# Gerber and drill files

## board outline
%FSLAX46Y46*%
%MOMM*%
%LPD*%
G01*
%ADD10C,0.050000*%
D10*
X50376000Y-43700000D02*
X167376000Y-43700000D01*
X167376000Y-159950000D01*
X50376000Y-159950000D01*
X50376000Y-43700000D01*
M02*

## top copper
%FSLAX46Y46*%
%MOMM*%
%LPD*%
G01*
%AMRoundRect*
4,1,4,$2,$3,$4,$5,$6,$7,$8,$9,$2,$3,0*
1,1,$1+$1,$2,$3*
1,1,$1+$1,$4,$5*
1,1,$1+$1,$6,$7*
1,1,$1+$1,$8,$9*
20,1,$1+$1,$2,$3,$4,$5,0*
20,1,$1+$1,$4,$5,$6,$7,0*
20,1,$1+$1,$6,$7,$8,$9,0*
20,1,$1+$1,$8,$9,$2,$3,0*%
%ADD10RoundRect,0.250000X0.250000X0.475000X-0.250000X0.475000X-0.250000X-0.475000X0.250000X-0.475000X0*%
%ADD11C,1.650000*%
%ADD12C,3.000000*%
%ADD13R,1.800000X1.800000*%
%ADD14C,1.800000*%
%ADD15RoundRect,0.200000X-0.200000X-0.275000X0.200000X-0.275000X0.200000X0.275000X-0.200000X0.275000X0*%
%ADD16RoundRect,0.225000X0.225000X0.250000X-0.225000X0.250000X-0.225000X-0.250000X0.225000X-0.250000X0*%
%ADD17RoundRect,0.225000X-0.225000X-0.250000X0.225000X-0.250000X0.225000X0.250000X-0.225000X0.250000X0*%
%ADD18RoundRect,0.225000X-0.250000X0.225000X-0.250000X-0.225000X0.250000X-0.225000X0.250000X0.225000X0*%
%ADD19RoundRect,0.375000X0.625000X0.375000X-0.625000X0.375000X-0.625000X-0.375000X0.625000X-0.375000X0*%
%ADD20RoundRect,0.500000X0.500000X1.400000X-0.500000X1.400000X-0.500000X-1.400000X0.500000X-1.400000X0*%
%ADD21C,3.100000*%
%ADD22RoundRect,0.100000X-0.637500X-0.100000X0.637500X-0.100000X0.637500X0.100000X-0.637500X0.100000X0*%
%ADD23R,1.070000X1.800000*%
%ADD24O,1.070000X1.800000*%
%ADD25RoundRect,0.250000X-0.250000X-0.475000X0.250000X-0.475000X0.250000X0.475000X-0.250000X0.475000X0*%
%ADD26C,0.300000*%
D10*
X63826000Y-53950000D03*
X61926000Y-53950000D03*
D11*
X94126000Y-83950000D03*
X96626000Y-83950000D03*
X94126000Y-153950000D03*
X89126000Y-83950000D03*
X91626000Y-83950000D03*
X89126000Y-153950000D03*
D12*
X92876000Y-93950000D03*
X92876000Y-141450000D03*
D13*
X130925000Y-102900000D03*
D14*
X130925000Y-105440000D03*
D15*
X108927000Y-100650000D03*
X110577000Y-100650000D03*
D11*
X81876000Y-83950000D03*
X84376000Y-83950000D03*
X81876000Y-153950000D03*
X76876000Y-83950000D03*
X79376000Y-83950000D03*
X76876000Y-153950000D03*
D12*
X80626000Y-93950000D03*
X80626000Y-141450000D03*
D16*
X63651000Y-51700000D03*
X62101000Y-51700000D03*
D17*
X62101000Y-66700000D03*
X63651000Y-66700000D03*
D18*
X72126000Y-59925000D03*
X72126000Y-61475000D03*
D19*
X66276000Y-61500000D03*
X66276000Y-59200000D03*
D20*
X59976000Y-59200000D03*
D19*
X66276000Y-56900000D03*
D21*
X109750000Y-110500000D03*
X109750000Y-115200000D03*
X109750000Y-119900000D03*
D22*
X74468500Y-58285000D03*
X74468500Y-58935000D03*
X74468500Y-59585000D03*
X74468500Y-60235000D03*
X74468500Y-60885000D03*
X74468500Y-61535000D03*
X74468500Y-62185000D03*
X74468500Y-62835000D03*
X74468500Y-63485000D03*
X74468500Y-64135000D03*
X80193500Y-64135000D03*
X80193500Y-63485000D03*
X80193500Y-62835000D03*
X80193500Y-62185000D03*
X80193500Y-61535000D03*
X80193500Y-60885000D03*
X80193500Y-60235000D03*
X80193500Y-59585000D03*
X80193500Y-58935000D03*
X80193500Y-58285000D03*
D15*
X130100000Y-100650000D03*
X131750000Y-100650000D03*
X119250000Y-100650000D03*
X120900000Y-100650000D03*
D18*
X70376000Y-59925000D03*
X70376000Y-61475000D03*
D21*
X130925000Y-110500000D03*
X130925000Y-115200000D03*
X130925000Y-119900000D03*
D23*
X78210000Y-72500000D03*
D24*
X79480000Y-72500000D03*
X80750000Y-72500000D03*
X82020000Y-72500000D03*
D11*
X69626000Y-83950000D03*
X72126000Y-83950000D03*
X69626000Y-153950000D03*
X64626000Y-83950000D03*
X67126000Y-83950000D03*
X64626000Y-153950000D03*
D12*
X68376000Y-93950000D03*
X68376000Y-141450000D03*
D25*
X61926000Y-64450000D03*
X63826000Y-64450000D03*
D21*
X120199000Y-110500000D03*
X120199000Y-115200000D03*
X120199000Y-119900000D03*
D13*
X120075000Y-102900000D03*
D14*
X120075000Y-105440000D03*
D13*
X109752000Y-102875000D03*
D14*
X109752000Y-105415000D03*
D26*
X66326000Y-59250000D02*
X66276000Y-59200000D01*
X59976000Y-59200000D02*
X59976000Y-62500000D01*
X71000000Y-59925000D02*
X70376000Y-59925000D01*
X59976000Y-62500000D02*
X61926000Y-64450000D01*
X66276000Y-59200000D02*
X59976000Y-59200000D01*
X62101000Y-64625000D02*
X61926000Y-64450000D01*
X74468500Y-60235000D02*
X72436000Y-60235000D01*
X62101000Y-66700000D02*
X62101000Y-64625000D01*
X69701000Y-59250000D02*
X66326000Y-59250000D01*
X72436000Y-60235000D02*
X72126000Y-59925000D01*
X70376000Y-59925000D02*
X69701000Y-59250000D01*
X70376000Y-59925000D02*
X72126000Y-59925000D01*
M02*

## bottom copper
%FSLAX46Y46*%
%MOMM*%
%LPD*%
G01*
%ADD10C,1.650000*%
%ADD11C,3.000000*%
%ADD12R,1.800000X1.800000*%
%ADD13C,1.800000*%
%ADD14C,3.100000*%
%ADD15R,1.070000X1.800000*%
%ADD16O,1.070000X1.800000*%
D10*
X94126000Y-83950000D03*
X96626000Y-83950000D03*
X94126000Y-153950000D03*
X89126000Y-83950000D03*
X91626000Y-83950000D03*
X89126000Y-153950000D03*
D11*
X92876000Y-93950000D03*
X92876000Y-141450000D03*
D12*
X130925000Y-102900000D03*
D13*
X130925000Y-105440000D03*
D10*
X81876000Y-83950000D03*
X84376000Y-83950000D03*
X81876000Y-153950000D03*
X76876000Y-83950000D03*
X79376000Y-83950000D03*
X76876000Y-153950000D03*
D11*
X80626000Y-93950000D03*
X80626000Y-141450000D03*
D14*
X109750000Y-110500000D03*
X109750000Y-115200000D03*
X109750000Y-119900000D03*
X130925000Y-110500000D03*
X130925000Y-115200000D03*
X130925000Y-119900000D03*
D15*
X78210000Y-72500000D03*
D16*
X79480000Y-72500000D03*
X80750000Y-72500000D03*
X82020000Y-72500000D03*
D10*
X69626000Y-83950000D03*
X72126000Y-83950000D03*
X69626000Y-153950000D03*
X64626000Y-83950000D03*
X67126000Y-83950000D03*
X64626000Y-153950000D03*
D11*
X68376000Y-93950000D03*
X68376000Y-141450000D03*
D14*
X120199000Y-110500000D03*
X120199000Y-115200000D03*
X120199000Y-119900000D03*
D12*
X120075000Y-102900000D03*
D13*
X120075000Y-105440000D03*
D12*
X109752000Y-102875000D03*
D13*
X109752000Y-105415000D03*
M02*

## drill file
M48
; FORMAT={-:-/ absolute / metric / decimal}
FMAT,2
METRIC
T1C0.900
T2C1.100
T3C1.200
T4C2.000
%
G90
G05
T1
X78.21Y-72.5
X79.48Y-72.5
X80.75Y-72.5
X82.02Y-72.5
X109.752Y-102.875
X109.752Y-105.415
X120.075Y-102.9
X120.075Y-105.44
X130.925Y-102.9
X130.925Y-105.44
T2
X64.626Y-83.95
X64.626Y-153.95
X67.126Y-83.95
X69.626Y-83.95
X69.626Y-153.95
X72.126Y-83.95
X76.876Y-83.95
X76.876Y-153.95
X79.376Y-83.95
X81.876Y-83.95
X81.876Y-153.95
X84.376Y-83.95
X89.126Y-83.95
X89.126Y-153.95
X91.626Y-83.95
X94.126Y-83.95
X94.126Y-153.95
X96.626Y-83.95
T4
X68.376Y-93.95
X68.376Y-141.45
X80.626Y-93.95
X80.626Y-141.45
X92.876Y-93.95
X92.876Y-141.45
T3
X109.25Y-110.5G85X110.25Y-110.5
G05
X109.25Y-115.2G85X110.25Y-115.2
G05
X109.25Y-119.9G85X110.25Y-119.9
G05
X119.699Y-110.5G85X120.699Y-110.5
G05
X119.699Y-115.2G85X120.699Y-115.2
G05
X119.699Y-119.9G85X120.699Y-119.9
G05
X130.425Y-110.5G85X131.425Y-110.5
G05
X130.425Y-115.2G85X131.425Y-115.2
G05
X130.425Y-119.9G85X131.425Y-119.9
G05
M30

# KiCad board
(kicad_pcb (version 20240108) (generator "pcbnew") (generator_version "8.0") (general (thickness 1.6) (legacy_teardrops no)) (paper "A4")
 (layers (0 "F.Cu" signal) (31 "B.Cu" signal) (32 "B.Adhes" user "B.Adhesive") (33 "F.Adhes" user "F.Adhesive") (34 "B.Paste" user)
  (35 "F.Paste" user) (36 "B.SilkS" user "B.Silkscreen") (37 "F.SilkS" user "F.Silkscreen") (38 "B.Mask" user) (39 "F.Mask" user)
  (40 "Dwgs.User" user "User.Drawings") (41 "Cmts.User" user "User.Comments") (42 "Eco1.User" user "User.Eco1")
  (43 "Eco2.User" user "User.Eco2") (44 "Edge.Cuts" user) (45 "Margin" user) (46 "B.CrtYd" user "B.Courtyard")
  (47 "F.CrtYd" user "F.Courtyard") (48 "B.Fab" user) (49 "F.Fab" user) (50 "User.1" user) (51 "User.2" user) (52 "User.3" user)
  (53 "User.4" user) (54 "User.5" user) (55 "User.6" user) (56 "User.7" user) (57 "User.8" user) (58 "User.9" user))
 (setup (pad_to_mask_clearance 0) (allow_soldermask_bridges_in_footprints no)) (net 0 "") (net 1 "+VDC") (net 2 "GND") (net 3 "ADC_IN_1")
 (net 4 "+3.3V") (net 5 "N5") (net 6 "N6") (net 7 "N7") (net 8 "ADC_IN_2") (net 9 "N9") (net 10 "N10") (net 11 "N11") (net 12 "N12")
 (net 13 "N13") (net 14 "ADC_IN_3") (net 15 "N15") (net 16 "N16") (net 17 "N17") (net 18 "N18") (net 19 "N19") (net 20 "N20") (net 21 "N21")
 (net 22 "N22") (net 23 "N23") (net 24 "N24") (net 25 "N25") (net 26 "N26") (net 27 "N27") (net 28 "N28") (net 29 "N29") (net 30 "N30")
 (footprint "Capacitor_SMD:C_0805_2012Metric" (layer "F.Cu") (at 62.876 53.95 180)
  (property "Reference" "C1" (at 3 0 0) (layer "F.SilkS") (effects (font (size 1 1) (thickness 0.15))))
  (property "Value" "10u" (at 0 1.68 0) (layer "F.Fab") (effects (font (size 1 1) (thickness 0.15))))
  (pad "1" smd roundrect (at -0.95 0 180) (size 1 1.45) (layers "F.Cu" "F.Paste" "F.Mask") (roundrect_rratio 0.25) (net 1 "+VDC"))
  (pad "2" smd roundrect (at 0.95 0 180) (size 1 1.45) (layers "F.Cu" "F.Paste" "F.Mask") (roundrect_rratio 0.25) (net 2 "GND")))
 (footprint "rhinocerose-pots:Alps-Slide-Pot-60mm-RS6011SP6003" (layer "F.Cu") (at 94.126 83.95 -90)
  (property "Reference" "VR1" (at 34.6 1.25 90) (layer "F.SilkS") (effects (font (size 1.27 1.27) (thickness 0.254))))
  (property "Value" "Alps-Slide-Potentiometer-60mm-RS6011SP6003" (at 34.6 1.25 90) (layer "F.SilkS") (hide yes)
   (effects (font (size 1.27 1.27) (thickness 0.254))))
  (pad "1" thru_hole circle (at 0 0 270) (size 1.65 1.65) (drill 1.1) (layers "*.Cu" "*.Mask") (remove_unused_layers no) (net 2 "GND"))
  (pad "2" thru_hole circle (at 0 -2.5 270) (size 1.65 1.65) (drill 1.1) (layers "*.Cu" "*.Mask") (remove_unused_layers no)
   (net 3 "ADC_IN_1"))
  (pad "3" thru_hole circle (at 70 0 270) (size 1.65 1.65) (drill 1.1) (layers "*.Cu" "*.Mask") (remove_unused_layers no) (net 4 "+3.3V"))
  (pad "L1" thru_hole circle (at 0 5 270) (size 1.65 1.65) (drill 1.1) (layers "*.Cu" "*.Mask") (remove_unused_layers no) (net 2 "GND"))
  (pad "L2" thru_hole circle (at 0 2.5 270) (size 1.65 1.65) (drill 1.1) (layers "*.Cu" "*.Mask") (remove_unused_layers no) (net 2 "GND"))
  (pad "L3" thru_hole circle (at 70 5 270) (size 1.65 1.65) (drill 1.1) (layers "*.Cu" "*.Mask") (remove_unused_layers no) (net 2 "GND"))
  (pad "MH1" thru_hole circle (at 10 1.25 270) (size 3 3) (drill 2) (layers "*.Cu" "*.Mask") (remove_unused_layers no) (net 2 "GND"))
  (pad "MH2" thru_hole circle (at 57.5 1.25 270) (size 3 3) (drill 2) (layers "*.Cu" "*.Mask") (remove_unused_layers no) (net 2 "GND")))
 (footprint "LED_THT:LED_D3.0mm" (layer "F.Cu") (at 130.925 102.9 -90)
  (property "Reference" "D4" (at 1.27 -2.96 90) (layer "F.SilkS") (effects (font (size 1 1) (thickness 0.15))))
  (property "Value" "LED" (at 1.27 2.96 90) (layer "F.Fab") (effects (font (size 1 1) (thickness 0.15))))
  (pad "1" thru_hole rect (at 0 0 270) (size 1.8 1.8) (drill 0.9) (layers "*.Cu" "*.Mask") (remove_unused_layers no) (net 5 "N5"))
  (pad "2" thru_hole circle (at 2.54 0 270) (size 1.8 1.8) (drill 0.9) (layers "*.Cu" "*.Mask") (remove_unused_layers no) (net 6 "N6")))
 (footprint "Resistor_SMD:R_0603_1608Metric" (layer "F.Cu") (at 109.752 100.65)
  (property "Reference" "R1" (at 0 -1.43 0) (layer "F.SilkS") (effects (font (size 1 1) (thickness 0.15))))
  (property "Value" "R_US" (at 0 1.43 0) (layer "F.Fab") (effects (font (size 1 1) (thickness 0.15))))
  (pad "1" smd roundrect (at -0.825 0) (size 0.8 0.95) (layers "F.Cu" "F.Paste" "F.Mask") (roundrect_rratio 0.25) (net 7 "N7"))
  (pad "2" smd roundrect (at 0.825 0) (size 0.8 0.95) (layers "F.Cu" "F.Paste" "F.Mask") (roundrect_rratio 0.25) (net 2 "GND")))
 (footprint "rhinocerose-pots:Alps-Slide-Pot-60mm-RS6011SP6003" (layer "F.Cu") (at 81.876 83.95 -90)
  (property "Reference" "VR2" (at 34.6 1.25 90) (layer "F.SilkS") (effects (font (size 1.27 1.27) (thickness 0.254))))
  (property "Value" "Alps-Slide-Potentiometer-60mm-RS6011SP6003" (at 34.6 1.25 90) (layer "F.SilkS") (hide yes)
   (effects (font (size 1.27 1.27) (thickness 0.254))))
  (pad "1" thru_hole circle (at 0 0 270) (size 1.65 1.65) (drill 1.1) (layers "*.Cu" "*.Mask") (remove_unused_layers no) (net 2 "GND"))
  (pad "2" thru_hole circle (at 0 -2.5 270) (size 1.65 1.65) (drill 1.1) (layers "*.Cu" "*.Mask") (remove_unused_layers no)
   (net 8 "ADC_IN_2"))
  (pad "3" thru_hole circle (at 70 0 270) (size 1.65 1.65) (drill 1.1) (layers "*.Cu" "*.Mask") (remove_unused_layers no) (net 4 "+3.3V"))
  (pad "L1" thru_hole circle (at 0 5 270) (size 1.65 1.65) (drill 1.1) (layers "*.Cu" "*.Mask") (remove_unused_layers no) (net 2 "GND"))
  (pad "L2" thru_hole circle (at 0 2.5 270) (size 1.65 1.65) (drill 1.1) (layers "*.Cu" "*.Mask") (remove_unused_layers no) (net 2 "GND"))
  (pad "L3" thru_hole circle (at 70 5 270) (size 1.65 1.65) (drill 1.1) (layers "*.Cu" "*.Mask") (remove_unused_layers no) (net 2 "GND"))
  (pad "MH1" thru_hole circle (at 10 1.25 270) (size 3 3) (drill 2) (layers "*.Cu" "*.Mask") (remove_unused_layers no) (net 2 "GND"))
  (pad "MH2" thru_hole circle (at 57.5 1.25 270) (size 3 3) (drill 2) (layers "*.Cu" "*.Mask") (remove_unused_layers no) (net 2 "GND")))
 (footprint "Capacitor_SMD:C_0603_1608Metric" (layer "F.Cu") (at 62.876 51.7 180)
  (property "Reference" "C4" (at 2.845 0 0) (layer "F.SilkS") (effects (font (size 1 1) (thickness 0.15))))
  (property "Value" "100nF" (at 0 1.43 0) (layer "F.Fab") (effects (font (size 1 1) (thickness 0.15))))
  (pad "1" smd roundrect (at -0.775 0 180) (size 0.9 0.95) (layers "F.Cu" "F.Paste" "F.Mask") (roundrect_rratio 0.25) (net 1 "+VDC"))
  (pad "2" smd roundrect (at 0.775 0 180) (size 0.9 0.95) (layers "F.Cu" "F.Paste" "F.Mask") (roundrect_rratio 0.25) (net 2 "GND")))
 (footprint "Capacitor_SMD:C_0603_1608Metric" (layer "F.Cu") (at 62.876 66.7)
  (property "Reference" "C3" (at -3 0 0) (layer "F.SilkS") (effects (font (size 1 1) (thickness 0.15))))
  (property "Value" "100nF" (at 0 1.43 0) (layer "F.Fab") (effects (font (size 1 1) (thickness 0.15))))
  (pad "1" smd roundrect (at -0.775 0) (size 0.9 0.95) (layers "F.Cu" "F.Paste" "F.Mask") (roundrect_rratio 0.25) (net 4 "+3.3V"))
  (pad "2" smd roundrect (at 0.775 0) (size 0.9 0.95) (layers "F.Cu" "F.Paste" "F.Mask") (roundrect_rratio 0.25) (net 2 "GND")))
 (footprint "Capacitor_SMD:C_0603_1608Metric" (layer "F.Cu") (at 72.126 60.7 -90)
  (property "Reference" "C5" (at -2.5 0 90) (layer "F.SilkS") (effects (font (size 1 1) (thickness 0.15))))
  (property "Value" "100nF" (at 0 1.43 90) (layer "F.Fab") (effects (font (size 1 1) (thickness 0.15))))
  (pad "1" smd roundrect (at -0.775 0 270) (size 0.9 0.95) (layers "F.Cu" "F.Paste" "F.Mask") (roundrect_rratio 0.25) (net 4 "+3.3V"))
  (pad "2" smd roundrect (at 0.775 0 270) (size 0.9 0.95) (layers "F.Cu" "F.Paste" "F.Mask") (roundrect_rratio 0.25) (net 2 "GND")))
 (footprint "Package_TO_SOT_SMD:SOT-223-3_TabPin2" (layer "F.Cu") (at 63.126 59.2 180)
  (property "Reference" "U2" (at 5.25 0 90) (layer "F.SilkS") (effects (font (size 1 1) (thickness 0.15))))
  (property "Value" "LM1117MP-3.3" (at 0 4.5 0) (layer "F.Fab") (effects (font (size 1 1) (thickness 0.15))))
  (pad "1" smd roundrect (at -3.15 -2.3 180) (size 2 1.5) (layers "F.Cu" "F.Paste" "F.Mask") (roundrect_rratio 0.25) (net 2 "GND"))
  (pad "2" smd roundrect (at -3.15 0 180) (size 2 1.5) (layers "F.Cu" "F.Paste" "F.Mask") (roundrect_rratio 0.25) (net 4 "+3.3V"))
  (pad "2" smd roundrect (at 3.15 0 180) (size 2 3.8) (layers "F.Cu" "F.Paste" "F.Mask") (roundrect_rratio 0.25) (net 4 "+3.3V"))
  (pad "3" smd roundrect (at -3.15 2.3 180) (size 2 1.5) (layers "F.Cu" "F.Paste" "F.Mask") (roundrect_rratio 0.25) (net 1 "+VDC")))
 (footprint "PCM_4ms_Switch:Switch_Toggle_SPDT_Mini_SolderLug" (layer "F.Cu") (at 109.75 115.2)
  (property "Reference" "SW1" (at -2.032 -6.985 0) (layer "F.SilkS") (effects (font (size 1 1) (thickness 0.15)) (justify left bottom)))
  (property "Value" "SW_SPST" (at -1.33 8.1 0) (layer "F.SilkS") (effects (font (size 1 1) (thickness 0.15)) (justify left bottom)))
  (pad "1" thru_hole circle (at 0 -4.7) (size 3.1 3.1) (drill oval 2.2 1.2) (layers "*.Cu" "*.Mask") (remove_unused_layers no) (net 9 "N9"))
  (pad "2" thru_hole circle (at 0 0) (size 3.1 3.1) (drill oval 2.2 1.2) (layers "*.Cu" "*.Mask") (remove_unused_layers no) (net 4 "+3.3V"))
  (pad "3" thru_hole circle (at 0 4.7) (size 3.1 3.1) (drill oval 2.2 1.2) (layers "*.Cu" "*.Mask") (remove_unused_layers no)))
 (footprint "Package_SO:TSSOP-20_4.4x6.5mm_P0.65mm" (layer "F.Cu") (at 77.331 61.21)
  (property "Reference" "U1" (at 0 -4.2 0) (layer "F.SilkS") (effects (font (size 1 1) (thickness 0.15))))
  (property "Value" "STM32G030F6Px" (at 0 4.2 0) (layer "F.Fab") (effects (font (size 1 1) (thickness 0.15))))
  (pad "1" smd roundrect (at -2.8625 -2.925) (size 1.475 0.4) (layers "F.Cu" "F.Paste" "F.Mask") (roundrect_rratio 0.25) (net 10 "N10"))
  (pad "2" smd roundrect (at -2.8625 -2.275) (size 1.475 0.4) (layers "F.Cu" "F.Paste" "F.Mask") (roundrect_rratio 0.25) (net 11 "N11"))
  (pad "3" smd roundrect (at -2.8625 -1.625) (size 1.475 0.4) (layers "F.Cu" "F.Paste" "F.Mask") (roundrect_rratio 0.25) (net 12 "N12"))
  (pad "4" smd roundrect (at -2.8625 -0.975) (size 1.475 0.4) (layers "F.Cu" "F.Paste" "F.Mask") (roundrect_rratio 0.25) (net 4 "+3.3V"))
  (pad "5" smd roundrect (at -2.8625 -0.325) (size 1.475 0.4) (layers "F.Cu" "F.Paste" "F.Mask") (roundrect_rratio 0.25) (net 2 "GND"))
  (pad "6" smd roundrect (at -2.8625 0.325) (size 1.475 0.4) (layers "F.Cu" "F.Paste" "F.Mask") (roundrect_rratio 0.25) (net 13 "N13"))
  (pad "7" smd roundrect (at -2.8625 0.975) (size 1.475 0.4) (layers "F.Cu" "F.Paste" "F.Mask") (roundrect_rratio 0.25) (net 3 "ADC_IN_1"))
  (pad "8" smd roundrect (at -2.8625 1.625) (size 1.475 0.4) (layers "F.Cu" "F.Paste" "F.Mask") (roundrect_rratio 0.25) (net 8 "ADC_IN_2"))
  (pad "9" smd roundrect (at -2.8625 2.275) (size 1.475 0.4) (layers "F.Cu" "F.Paste" "F.Mask") (roundrect_rratio 0.25) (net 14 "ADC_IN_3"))
  (pad "10" smd roundrect (at -2.8625 2.925) (size 1.475 0.4) (layers "F.Cu" "F.Paste" "F.Mask") (roundrect_rratio 0.25) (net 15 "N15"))
  (pad "11" smd roundrect (at 2.8625 2.925) (size 1.475 0.4) (layers "F.Cu" "F.Paste" "F.Mask") (roundrect_rratio 0.25) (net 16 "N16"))
  (pad "12" smd roundrect (at 2.8625 2.275) (size 1.475 0.4) (layers "F.Cu" "F.Paste" "F.Mask") (roundrect_rratio 0.25) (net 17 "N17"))
  (pad "13" smd roundrect (at 2.8625 1.625) (size 1.475 0.4) (layers "F.Cu" "F.Paste" "F.Mask") (roundrect_rratio 0.25) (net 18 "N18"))
  (pad "14" smd roundrect (at 2.8625 0.975) (size 1.475 0.4) (layers "F.Cu" "F.Paste" "F.Mask") (roundrect_rratio 0.25) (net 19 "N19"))
  (pad "15" smd roundrect (at 2.8625 0.325) (size 1.475 0.4) (layers "F.Cu" "F.Paste" "F.Mask") (roundrect_rratio 0.25) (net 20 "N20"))
  (pad "16" smd roundrect (at 2.8625 -0.325) (size 1.475 0.4) (layers "F.Cu" "F.Paste" "F.Mask") (roundrect_rratio 0.25) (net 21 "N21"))
  (pad "17" smd roundrect (at 2.8625 -0.975) (size 1.475 0.4) (layers "F.Cu" "F.Paste" "F.Mask") (roundrect_rratio 0.25) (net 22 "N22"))
  (pad "18" smd roundrect (at 2.8625 -1.625) (size 1.475 0.4) (layers "F.Cu" "F.Paste" "F.Mask") (roundrect_rratio 0.25) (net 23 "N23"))
  (pad "19" smd roundrect (at 2.8625 -2.275) (size 1.475 0.4) (layers "F.Cu" "F.Paste" "F.Mask") (roundrect_rratio 0.25) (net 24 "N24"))
  (pad "20" smd roundrect (at 2.8625 -2.925) (size 1.475 0.4) (layers "F.Cu" "F.Paste" "F.Mask") (roundrect_rratio 0.25) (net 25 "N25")))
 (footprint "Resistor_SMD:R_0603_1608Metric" (layer "F.Cu") (at 130.925 100.65)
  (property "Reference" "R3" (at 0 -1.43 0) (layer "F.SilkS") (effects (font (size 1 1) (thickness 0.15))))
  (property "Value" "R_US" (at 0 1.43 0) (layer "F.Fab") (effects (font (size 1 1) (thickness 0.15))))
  (pad "1" smd roundrect (at -0.825 0) (size 0.8 0.95) (layers "F.Cu" "F.Paste" "F.Mask") (roundrect_rratio 0.25) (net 5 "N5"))
  (pad "2" smd roundrect (at 0.825 0) (size 0.8 0.95) (layers "F.Cu" "F.Paste" "F.Mask") (roundrect_rratio 0.25) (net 2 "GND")))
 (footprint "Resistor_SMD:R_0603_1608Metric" (layer "F.Cu") (at 120.075 100.65)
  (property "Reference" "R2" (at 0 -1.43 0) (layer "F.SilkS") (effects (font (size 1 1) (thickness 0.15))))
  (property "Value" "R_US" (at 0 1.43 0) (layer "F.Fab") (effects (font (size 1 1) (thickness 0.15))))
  (pad "1" smd roundrect (at -0.825 0) (size 0.8 0.95) (layers "F.Cu" "F.Paste" "F.Mask") (roundrect_rratio 0.25) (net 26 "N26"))
  (pad "2" smd roundrect (at 0.825 0) (size 0.8 0.95) (layers "F.Cu" "F.Paste" "F.Mask") (roundrect_rratio 0.25) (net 2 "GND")))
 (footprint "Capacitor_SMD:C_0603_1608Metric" (layer "F.Cu") (at 70.376 60.7 -90)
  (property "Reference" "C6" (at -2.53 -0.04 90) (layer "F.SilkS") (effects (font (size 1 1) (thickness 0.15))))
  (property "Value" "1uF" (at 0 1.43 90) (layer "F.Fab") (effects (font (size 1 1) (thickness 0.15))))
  (pad "1" smd roundrect (at -0.775 0 270) (size 0.9 0.95) (layers "F.Cu" "F.Paste" "F.Mask") (roundrect_rratio 0.25) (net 4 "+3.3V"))
  (pad "2" smd roundrect (at 0.775 0 270) (size 0.9 0.95) (layers "F.Cu" "F.Paste" "F.Mask") (roundrect_rratio 0.25) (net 2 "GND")))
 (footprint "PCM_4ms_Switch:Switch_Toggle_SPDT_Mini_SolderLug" (layer "F.Cu") (at 130.925 115.2)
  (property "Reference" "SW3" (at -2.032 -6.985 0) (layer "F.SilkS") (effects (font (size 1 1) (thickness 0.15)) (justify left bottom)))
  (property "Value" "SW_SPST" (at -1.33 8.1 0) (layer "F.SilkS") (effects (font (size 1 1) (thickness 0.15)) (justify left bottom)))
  (pad "1" thru_hole circle (at 0 -4.7) (size 3.1 3.1) (drill oval 2.2 1.2) (layers "*.Cu" "*.Mask") (remove_unused_layers no) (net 6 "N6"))
  (pad "2" thru_hole circle (at 0 0) (size 3.1 3.1) (drill oval 2.2 1.2) (layers "*.Cu" "*.Mask") (remove_unused_layers no) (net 4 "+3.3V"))
  (pad "3" thru_hole circle (at 0 4.7) (size 3.1 3.1) (drill oval 2.2 1.2) (layers "*.Cu" "*.Mask") (remove_unused_layers no)))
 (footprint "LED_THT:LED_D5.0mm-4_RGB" (layer "F.Cu") (at 78.21 72.5)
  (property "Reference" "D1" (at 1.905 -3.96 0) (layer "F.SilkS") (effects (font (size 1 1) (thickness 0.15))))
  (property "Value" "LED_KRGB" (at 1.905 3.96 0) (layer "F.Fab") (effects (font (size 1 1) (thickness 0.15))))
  (pad "1" thru_hole rect (at 0 0) (size 1.07 1.8) (drill 0.9) (layers "*.Cu" "*.Mask") (remove_unused_layers no) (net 2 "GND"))
  (pad "2" thru_hole oval (at 1.27 0) (size 1.07 1.8) (drill 0.9) (layers "*.Cu" "*.Mask") (remove_unused_layers no) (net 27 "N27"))
  (pad "3" thru_hole oval (at 2.54 0) (size 1.07 1.8) (drill 0.9) (layers "*.Cu" "*.Mask") (remove_unused_layers no) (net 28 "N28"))
  (pad "4" thru_hole oval (at 3.81 0) (size 1.07 1.8) (drill 0.9) (layers "*.Cu" "*.Mask") (remove_unused_layers no) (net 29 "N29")))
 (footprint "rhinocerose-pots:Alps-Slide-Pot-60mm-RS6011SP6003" (layer "F.Cu") (at 69.626 83.95 -90)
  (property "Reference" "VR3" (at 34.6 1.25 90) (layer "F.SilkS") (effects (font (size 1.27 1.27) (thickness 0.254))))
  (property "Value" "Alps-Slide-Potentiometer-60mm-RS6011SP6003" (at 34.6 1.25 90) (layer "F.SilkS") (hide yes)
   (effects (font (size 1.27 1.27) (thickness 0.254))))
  (pad "1" thru_hole circle (at 0 0 270) (size 1.65 1.65) (drill 1.1) (layers "*.Cu" "*.Mask") (remove_unused_layers no) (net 2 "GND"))
  (pad "2" thru_hole circle (at 0 -2.5 270) (size 1.65 1.65) (drill 1.1) (layers "*.Cu" "*.Mask") (remove_unused_layers no)
   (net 14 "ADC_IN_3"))
  (pad "3" thru_hole circle (at 70 0 270) (size 1.65 1.65) (drill 1.1) (layers "*.Cu" "*.Mask") (remove_unused_layers no) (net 4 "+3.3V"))
  (pad "L1" thru_hole circle (at 0 5 270) (size 1.65 1.65) (drill 1.1) (layers "*.Cu" "*.Mask") (remove_unused_layers no) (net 2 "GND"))
  (pad "L2" thru_hole circle (at 0 2.5 270) (size 1.65 1.65) (drill 1.1) (layers "*.Cu" "*.Mask") (remove_unused_layers no) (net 2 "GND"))
  (pad "L3" thru_hole circle (at 70 5 270) (size 1.65 1.65) (drill 1.1) (layers "*.Cu" "*.Mask") (remove_unused_layers no) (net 2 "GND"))
  (pad "MH1" thru_hole circle (at 10 1.25 270) (size 3 3) (drill 2) (layers "*.Cu" "*.Mask") (remove_unused_layers no) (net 2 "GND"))
  (pad "MH2" thru_hole circle (at 57.5 1.25 270) (size 3 3) (drill 2) (layers "*.Cu" "*.Mask") (remove_unused_layers no) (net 2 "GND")))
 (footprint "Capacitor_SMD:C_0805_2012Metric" (layer "F.Cu") (at 62.876 64.45)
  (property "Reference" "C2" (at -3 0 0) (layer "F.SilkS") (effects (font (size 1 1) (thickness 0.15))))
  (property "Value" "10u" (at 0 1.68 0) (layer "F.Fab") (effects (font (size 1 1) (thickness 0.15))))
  (pad "1" smd roundrect (at -0.95 0) (size 1 1.45) (layers "F.Cu" "F.Paste" "F.Mask") (roundrect_rratio 0.25) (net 4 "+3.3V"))
  (pad "2" smd roundrect (at 0.95 0) (size 1 1.45) (layers "F.Cu" "F.Paste" "F.Mask") (roundrect_rratio 0.25) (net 2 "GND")))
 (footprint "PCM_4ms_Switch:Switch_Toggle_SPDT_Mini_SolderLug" (layer "F.Cu") (at 120.199 115.2)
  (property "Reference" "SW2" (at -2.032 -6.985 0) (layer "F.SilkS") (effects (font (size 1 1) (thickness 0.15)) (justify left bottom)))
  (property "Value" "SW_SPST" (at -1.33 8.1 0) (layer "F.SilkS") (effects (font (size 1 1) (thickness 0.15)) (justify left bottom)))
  (pad "1" thru_hole circle (at 0 -4.7) (size 3.1 3.1) (drill oval 2.2 1.2) (layers "*.Cu" "*.Mask") (remove_unused_layers no)
   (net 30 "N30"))
  (pad "2" thru_hole circle (at 0 0) (size 3.1 3.1) (drill oval 2.2 1.2) (layers "*.Cu" "*.Mask") (remove_unused_layers no) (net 4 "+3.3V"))
  (pad "3" thru_hole circle (at 0 4.7) (size 3.1 3.1) (drill oval 2.2 1.2) (layers "*.Cu" "*.Mask") (remove_unused_layers no)))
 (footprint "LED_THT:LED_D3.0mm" (layer "F.Cu") (at 120.075 102.9 -90)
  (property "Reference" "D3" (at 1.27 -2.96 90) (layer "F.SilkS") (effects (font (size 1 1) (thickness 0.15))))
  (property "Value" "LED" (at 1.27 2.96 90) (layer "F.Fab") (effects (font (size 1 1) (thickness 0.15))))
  (pad "1" thru_hole rect (at 0 0 270) (size 1.8 1.8) (drill 0.9) (layers "*.Cu" "*.Mask") (remove_unused_layers no) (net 26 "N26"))
  (pad "2" thru_hole circle (at 2.54 0 270) (size 1.8 1.8) (drill 0.9) (layers "*.Cu" "*.Mask") (remove_unused_layers no) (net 30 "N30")))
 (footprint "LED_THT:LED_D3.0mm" (layer "F.Cu") (at 109.752 102.875 -90)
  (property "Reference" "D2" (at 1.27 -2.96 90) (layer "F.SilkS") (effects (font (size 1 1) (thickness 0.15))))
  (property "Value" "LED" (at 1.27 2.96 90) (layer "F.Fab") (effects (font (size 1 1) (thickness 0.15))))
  (pad "1" thru_hole rect (at 0 0 270) (size 1.8 1.8) (drill 0.9) (layers "*.Cu" "*.Mask") (remove_unused_layers no) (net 7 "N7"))
  (pad "2" thru_hole circle (at 2.54 0 270) (size 1.8 1.8) (drill 0.9) (layers "*.Cu" "*.Mask") (remove_unused_layers no) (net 9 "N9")))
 (gr_rect (start 50.376 43.7) (end 167.376 159.95) (stroke (width 0.05) (type default)) (fill none) (layer "Edge.Cuts"))
 (segment (start 66.326 59.25) (end 66.276 59.2) (width 0.3) (layer "F.Cu") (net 4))
 (segment (start 59.976 59.2) (end 59.976 62.5) (width 0.3) (layer "F.Cu") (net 4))
 (segment (start 71 59.925) (end 70.376 59.925) (width 0.3) (layer "F.Cu") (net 4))
 (segment (start 59.976 62.5) (end 61.926 64.45) (width 0.3) (layer "F.Cu") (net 4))
 (segment (start 66.276 59.2) (end 59.976 59.2) (width 0.3) (layer "F.Cu") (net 4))
 (segment (start 62.101 64.625) (end 61.926 64.45) (width 0.3) (layer "F.Cu") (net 4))
 (segment (start 74.4685 60.235) (end 72.436 60.235) (width 0.3) (layer "F.Cu") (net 4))
 (segment (start 62.101 66.7) (end 62.101 64.625) (width 0.3) (layer "F.Cu") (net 4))
 (segment (start 69.701 59.25) (end 66.326 59.25) (width 0.3) (layer "F.Cu") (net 4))
 (segment (start 72.436 60.235) (end 72.126 59.925) (width 0.3) (layer "F.Cu") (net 4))
 (segment (start 70.376 59.925) (end 69.701 59.25) (width 0.3) (layer "F.Cu") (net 4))
 (segment (start 70.376 59.925) (end 72.126 59.925) (width 0.3) (layer "F.Cu") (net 4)))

